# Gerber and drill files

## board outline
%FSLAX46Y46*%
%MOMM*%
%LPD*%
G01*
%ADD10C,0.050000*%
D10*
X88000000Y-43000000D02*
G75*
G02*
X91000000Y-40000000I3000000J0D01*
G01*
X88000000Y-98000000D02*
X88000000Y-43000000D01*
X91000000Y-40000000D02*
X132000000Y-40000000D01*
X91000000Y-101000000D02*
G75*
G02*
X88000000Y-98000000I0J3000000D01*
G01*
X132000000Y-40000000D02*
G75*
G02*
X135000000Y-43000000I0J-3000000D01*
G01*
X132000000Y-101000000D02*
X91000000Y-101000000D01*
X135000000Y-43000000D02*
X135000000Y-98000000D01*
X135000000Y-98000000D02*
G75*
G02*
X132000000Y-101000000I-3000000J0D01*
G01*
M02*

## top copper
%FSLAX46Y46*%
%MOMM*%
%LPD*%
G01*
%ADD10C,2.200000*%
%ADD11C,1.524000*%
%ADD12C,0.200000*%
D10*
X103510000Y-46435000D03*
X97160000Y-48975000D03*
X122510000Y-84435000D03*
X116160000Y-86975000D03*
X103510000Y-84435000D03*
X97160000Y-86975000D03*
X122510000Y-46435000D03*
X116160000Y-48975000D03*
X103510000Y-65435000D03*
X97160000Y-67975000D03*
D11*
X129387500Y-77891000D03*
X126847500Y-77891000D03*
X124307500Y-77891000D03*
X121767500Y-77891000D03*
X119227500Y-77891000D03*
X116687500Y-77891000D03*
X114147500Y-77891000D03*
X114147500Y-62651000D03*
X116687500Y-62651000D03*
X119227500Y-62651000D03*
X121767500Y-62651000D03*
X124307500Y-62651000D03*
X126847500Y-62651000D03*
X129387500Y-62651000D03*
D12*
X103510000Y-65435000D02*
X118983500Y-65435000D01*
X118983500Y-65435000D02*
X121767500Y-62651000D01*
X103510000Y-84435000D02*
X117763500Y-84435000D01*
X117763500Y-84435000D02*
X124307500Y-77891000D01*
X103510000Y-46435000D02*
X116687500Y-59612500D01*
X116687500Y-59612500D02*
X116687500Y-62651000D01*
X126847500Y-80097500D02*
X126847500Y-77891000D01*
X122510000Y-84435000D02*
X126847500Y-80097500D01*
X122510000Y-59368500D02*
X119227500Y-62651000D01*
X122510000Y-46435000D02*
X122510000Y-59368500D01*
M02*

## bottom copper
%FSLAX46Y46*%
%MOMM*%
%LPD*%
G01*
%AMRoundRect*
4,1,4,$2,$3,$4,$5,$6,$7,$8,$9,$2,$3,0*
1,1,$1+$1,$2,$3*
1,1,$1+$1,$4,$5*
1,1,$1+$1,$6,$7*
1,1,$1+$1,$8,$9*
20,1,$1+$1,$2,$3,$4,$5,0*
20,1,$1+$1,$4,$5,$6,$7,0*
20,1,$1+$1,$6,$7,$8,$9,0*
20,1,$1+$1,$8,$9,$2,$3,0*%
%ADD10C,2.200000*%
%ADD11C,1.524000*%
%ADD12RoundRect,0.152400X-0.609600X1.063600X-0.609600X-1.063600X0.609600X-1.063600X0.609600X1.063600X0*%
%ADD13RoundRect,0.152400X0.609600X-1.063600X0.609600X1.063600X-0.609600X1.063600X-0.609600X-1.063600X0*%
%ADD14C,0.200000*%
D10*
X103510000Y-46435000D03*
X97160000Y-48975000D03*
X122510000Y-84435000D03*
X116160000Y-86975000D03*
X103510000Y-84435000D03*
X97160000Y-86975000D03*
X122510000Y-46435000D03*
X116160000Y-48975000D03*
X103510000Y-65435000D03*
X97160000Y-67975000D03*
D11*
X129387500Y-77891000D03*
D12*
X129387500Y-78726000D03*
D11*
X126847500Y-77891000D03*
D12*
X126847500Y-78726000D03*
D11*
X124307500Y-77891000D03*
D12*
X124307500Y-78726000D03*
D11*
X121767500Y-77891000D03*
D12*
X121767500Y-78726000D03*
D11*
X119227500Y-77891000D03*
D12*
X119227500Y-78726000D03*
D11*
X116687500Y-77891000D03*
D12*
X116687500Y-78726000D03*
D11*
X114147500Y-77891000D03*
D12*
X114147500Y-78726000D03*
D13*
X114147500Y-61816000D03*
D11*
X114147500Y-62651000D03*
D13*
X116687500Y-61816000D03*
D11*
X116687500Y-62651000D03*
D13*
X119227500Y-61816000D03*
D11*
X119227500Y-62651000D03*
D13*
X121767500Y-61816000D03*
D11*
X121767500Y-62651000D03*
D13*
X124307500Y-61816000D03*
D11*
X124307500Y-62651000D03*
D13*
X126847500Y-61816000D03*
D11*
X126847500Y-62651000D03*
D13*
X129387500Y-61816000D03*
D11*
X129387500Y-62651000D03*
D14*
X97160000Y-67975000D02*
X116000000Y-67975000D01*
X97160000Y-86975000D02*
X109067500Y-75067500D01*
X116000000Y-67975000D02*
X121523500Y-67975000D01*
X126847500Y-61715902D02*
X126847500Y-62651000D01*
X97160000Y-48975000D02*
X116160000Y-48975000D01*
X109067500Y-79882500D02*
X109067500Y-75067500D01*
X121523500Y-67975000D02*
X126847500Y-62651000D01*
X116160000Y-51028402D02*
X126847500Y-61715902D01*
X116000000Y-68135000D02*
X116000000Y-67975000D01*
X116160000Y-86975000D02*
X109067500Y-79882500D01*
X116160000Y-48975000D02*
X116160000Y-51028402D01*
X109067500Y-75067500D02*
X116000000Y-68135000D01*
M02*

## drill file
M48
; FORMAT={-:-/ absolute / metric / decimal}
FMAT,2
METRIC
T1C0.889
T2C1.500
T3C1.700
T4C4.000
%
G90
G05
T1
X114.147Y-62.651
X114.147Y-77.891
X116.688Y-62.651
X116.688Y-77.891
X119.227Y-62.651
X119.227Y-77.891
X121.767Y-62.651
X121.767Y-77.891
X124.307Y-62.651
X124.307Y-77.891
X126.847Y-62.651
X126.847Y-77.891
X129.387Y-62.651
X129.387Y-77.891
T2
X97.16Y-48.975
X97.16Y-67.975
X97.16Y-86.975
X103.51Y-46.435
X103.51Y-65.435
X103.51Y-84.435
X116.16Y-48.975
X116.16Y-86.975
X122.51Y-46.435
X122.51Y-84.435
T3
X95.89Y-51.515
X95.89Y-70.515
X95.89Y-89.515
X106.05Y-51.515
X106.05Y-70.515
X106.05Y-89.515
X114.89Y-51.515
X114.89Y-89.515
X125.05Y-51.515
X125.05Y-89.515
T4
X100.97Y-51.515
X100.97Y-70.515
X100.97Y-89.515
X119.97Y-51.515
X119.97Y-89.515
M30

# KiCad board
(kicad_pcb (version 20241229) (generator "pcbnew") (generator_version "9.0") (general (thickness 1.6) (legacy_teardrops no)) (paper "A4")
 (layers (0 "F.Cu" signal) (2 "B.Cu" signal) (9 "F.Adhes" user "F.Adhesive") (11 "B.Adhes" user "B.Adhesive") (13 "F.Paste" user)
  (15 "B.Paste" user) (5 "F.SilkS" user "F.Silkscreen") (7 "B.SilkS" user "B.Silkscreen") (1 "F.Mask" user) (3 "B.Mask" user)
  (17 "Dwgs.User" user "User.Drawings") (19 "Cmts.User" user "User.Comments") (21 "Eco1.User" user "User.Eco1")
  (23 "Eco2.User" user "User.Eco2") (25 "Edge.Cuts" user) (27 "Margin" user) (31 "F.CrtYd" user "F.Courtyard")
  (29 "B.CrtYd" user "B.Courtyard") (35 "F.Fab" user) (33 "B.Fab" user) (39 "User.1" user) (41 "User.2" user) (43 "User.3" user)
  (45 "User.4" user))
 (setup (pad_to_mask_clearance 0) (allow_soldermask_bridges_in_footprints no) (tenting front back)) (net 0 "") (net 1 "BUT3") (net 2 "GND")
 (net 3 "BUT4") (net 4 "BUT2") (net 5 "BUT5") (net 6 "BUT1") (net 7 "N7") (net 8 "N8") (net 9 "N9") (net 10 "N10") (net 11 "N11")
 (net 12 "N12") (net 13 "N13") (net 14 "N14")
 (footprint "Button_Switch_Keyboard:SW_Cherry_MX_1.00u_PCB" (layer "F.Cu") (at 103.51 46.435)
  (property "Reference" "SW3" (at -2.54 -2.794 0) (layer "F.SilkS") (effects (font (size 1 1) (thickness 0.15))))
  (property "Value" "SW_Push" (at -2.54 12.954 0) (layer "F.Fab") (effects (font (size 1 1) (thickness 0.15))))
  (pad "" np_thru_hole circle (at -7.62 5.08) (size 1.7 1.7) (drill 1.7) (layers "*.Cu" "*.Mask"))
  (pad "" np_thru_hole circle (at -2.54 5.08) (size 4 4) (drill 4) (layers "*.Cu" "*.Mask"))
  (pad "" np_thru_hole circle (at 2.54 5.08) (size 1.7 1.7) (drill 1.7) (layers "*.Cu" "*.Mask"))
  (pad "1" thru_hole circle (at 0 0) (size 2.2 2.2) (drill 1.5) (layers "*.Cu" "*.Mask") (remove_unused_layers no) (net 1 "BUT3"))
  (pad "2" thru_hole circle (at -6.35 2.54) (size 2.2 2.2) (drill 1.5) (layers "*.Cu" "*.Mask") (remove_unused_layers no) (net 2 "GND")))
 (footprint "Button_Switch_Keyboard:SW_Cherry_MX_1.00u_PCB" (layer "F.Cu") (at 122.51 84.435)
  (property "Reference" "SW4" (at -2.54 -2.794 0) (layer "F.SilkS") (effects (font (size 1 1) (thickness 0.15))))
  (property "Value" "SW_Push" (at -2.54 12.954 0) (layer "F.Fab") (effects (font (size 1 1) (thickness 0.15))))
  (pad "" np_thru_hole circle (at -7.62 5.08) (size 1.7 1.7) (drill 1.7) (layers "*.Cu" "*.Mask"))
  (pad "" np_thru_hole circle (at -2.54 5.08) (size 4 4) (drill 4) (layers "*.Cu" "*.Mask"))
  (pad "" np_thru_hole circle (at 2.54 5.08) (size 1.7 1.7) (drill 1.7) (layers "*.Cu" "*.Mask"))
  (pad "1" thru_hole circle (at 0 0) (size 2.2 2.2) (drill 1.5) (layers "*.Cu" "*.Mask") (remove_unused_layers no) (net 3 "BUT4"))
  (pad "2" thru_hole circle (at -6.35 2.54) (size 2.2 2.2) (drill 1.5) (layers "*.Cu" "*.Mask") (remove_unused_layers no) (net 2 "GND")))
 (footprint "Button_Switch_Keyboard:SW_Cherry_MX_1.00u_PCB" (layer "F.Cu") (at 103.51 84.435)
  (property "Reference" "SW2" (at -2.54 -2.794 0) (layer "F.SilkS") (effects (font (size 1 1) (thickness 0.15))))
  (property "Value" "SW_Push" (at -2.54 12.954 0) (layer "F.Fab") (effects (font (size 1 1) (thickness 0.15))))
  (pad "" np_thru_hole circle (at -7.62 5.08) (size 1.7 1.7) (drill 1.7) (layers "*.Cu" "*.Mask"))
  (pad "" np_thru_hole circle (at -2.54 5.08) (size 4 4) (drill 4) (layers "*.Cu" "*.Mask"))
  (pad "" np_thru_hole circle (at 2.54 5.08) (size 1.7 1.7) (drill 1.7) (layers "*.Cu" "*.Mask"))
  (pad "1" thru_hole circle (at 0 0) (size 2.2 2.2) (drill 1.5) (layers "*.Cu" "*.Mask") (remove_unused_layers no) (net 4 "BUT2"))
  (pad "2" thru_hole circle (at -6.35 2.54) (size 2.2 2.2) (drill 1.5) (layers "*.Cu" "*.Mask") (remove_unused_layers no) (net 2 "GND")))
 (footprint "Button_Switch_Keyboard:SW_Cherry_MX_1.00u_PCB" (layer "F.Cu") (at 122.51 46.435)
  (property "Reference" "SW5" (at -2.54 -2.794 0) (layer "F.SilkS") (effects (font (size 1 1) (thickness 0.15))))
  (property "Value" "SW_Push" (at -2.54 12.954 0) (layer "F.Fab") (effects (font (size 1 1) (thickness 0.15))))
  (pad "" np_thru_hole circle (at -7.62 5.08) (size 1.7 1.7) (drill 1.7) (layers "*.Cu" "*.Mask"))
  (pad "" np_thru_hole circle (at -2.54 5.08) (size 4 4) (drill 4) (layers "*.Cu" "*.Mask"))
  (pad "" np_thru_hole circle (at 2.54 5.08) (size 1.7 1.7) (drill 1.7) (layers "*.Cu" "*.Mask"))
  (pad "1" thru_hole circle (at 0 0) (size 2.2 2.2) (drill 1.5) (layers "*.Cu" "*.Mask") (remove_unused_layers no) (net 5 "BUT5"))
  (pad "2" thru_hole circle (at -6.35 2.54) (size 2.2 2.2) (drill 1.5) (layers "*.Cu" "*.Mask") (remove_unused_layers no) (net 2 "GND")))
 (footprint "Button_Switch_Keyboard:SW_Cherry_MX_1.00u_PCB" (layer "F.Cu") (at 103.51 65.435)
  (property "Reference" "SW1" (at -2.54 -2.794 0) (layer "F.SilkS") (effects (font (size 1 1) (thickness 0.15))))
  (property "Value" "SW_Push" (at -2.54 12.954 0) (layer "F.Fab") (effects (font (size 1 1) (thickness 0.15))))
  (pad "" np_thru_hole circle (at -7.62 5.08) (size 1.7 1.7) (drill 1.7) (layers "*.Cu" "*.Mask"))
  (pad "" np_thru_hole circle (at -2.54 5.08) (size 4 4) (drill 4) (layers "*.Cu" "*.Mask"))
  (pad "" np_thru_hole circle (at 2.54 5.08) (size 1.7 1.7) (drill 1.7) (layers "*.Cu" "*.Mask"))
  (pad "1" thru_hole circle (at 0 0) (size 2.2 2.2) (drill 1.5) (layers "*.Cu" "*.Mask") (remove_unused_layers no) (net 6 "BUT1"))
  (pad "2" thru_hole circle (at -6.35 2.54) (size 2.2 2.2) (drill 1.5) (layers "*.Cu" "*.Mask") (remove_unused_layers no) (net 2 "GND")))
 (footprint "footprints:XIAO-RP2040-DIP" (layer "B.Cu") (at 121.7675 70.271)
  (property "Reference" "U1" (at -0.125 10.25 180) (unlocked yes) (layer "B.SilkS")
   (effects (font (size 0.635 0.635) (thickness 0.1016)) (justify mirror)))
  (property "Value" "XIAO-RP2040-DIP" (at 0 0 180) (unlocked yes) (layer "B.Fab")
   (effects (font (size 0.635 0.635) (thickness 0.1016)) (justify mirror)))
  (pad "1" thru_hole circle (at 7.62 7.62 270) (size 1.524 1.524) (drill 0.889) (layers "*.Cu" "*.Mask") (remove_unused_layers no)
   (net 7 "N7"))
  (pad "1" smd roundrect (at 7.62 8.455 270) (size 2.432 1.524) (layers "B.Cu" "B.Mask") (roundrect_rratio 0.1) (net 7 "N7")
   (thermal_bridge_angle 45))
  (pad "2" thru_hole circle (at 5.08 7.62 270) (size 1.524 1.524) (drill 0.889) (layers "*.Cu" "*.Mask") (remove_unused_layers no)
   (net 3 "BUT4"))
  (pad "2" smd roundrect (at 5.08 8.455 270) (size 2.432 1.524) (layers "B.Cu" "B.Mask") (roundrect_rratio 0.1) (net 3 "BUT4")
   (thermal_bridge_angle 45))
  (pad "3" thru_hole circle (at 2.54 7.62 270) (size 1.524 1.524) (drill 0.889) (layers "*.Cu" "*.Mask") (remove_unused_layers no)
   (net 4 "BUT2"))
  (pad "3" smd roundrect (at 2.54 8.455 270) (size 2.432 1.524) (layers "B.Cu" "B.Mask") (roundrect_rratio 0.1) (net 4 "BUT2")
   (thermal_bridge_angle 45))
  (pad "4" thru_hole circle (at 0 7.62 270) (size 1.524 1.524) (drill 0.889) (layers "*.Cu" "*.Mask") (remove_unused_layers no) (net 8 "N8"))
  (pad "4" smd roundrect (at 0 8.455 270) (size 2.432 1.524) (layers "B.Cu" "B.Mask") (roundrect_rratio 0.1) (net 8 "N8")
   (thermal_bridge_angle 45))
  (pad "5" thru_hole circle (at -2.54 7.62 270) (size 1.524 1.524) (drill 0.889) (layers "*.Cu" "*.Mask") (remove_unused_layers no)
   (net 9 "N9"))
  (pad "5" smd roundrect (at -2.54 8.455 270) (size 2.432 1.524) (layers "B.Cu" "B.Mask") (roundrect_rratio 0.1) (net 9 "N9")
   (thermal_bridge_angle 45))
  (pad "6" thru_hole circle (at -5.08 7.62 270) (size 1.524 1.524) (drill 0.889) (layers "*.Cu" "*.Mask") (remove_unused_layers no)
   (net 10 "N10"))
  (pad "6" smd roundrect (at -5.08 8.455 270) (size 2.432 1.524) (layers "B.Cu" "B.Mask") (roundrect_rratio 0.1) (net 10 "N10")
   (thermal_bridge_angle 45))
  (pad "7" thru_hole circle (at -7.62 7.62 270) (size 1.524 1.524) (drill 0.889) (layers "*.Cu" "*.Mask") (remove_unused_layers no)
   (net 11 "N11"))
  (pad "7" smd roundrect (at -7.62 8.455 270) (size 2.432 1.524) (layers "B.Cu" "B.Mask") (roundrect_rratio 0.1) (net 11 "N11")
   (thermal_bridge_angle 45))
  (pad "8" smd roundrect (at -7.62 -8.455 90) (size 2.432 1.524) (layers "B.Cu" "B.Mask") (roundrect_rratio 0.1) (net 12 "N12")
   (thermal_bridge_angle 45))
  (pad "8" thru_hole circle (at -7.62 -7.62 90) (size 1.524 1.524) (drill 0.889) (layers "*.Cu" "*.Mask") (remove_unused_layers no)
   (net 12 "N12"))
  (pad "9" smd roundrect (at -5.08 -8.455 90) (size 2.432 1.524) (layers "B.Cu" "B.Mask") (roundrect_rratio 0.1) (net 1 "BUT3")
   (thermal_bridge_angle 45))
  (pad "9" thru_hole circle (at -5.08 -7.62 90) (size 1.524 1.524) (drill 0.889) (layers "*.Cu" "*.Mask") (remove_unused_layers no)
   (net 1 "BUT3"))
  (pad "10" smd roundrect (at -2.54 -8.455 90) (size 2.432 1.524) (layers "B.Cu" "B.Mask") (roundrect_rratio 0.1) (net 5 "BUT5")
   (thermal_bridge_angle 45))
  (pad "10" thru_hole circle (at -2.54 -7.62 90) (size 1.524 1.524) (drill 0.889) (layers "*.Cu" "*.Mask") (remove_unused_layers no)
   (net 5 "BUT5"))
  (pad "11" smd roundrect (at 0 -8.455 90) (size 2.432 1.524) (layers "B.Cu" "B.Mask") (roundrect_rratio 0.1) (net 6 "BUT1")
   (thermal_bridge_angle 45))
  (pad "11" thru_hole circle (at 0 -7.62 90) (size 1.524 1.524) (drill 0.889) (layers "*.Cu" "*.Mask") (remove_unused_layers no)
   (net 6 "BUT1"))
  (pad "12" smd roundrect (at 2.54 -8.455 90) (size 2.432 1.524) (layers "B.Cu" "B.Mask") (roundrect_rratio 0.1) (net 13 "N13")
   (thermal_bridge_angle 45))
  (pad "12" thru_hole circle (at 2.54 -7.62 90) (size 1.524 1.524) (drill 0.889) (layers "*.Cu" "*.Mask") (remove_unused_layers no)
   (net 13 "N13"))
  (pad "13" smd roundrect (at 5.08 -8.455 90) (size 2.432 1.524) (layers "B.Cu" "B.Mask") (roundrect_rratio 0.1) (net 2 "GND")
   (thermal_bridge_angle 45))
  (pad "13" thru_hole circle (at 5.08 -7.62 90) (size 1.524 1.524) (drill 0.889) (layers "*.Cu" "*.Mask") (remove_unused_layers no)
   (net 2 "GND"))
  (pad "14" smd roundrect (at 7.62 -8.455 90) (size 2.432 1.524) (layers "B.Cu" "B.Mask") (roundrect_rratio 0.1) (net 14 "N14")
   (thermal_bridge_angle 45))
  (pad "14" thru_hole circle (at 7.62 -7.62 90) (size 1.524 1.524) (drill 0.889) (layers "*.Cu" "*.Mask") (remove_unused_layers no)
   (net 14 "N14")))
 (gr_arc (start 88 43) (mid 88.87868 40.87868) (end 91 40) (stroke (width 0.05) (type default)) (layer "Edge.Cuts"))
 (gr_line (start 88 98) (end 88 43) (stroke (width 0.05) (type default)) (layer "Edge.Cuts"))
 (gr_line (start 91 40) (end 132 40) (stroke (width 0.05) (type default)) (layer "Edge.Cuts"))
 (gr_arc (start 91 101) (mid 88.87868 100.12132) (end 88 98) (stroke (width 0.05) (type default)) (layer "Edge.Cuts"))
 (gr_arc (start 132 40) (mid 134.12132 40.87868) (end 135 43) (stroke (width 0.05) (type default)) (layer "Edge.Cuts"))
 (gr_line (start 132 101) (end 91 101) (stroke (width 0.05) (type default)) (layer "Edge.Cuts"))
 (gr_line (start 135 43) (end 135 98) (stroke (width 0.05) (type default)) (layer "Edge.Cuts"))
 (gr_arc (start 135 98) (mid 134.12132 100.12132) (end 132 101) (stroke (width 0.05) (type default)) (layer "Edge.Cuts"))
 (segment (start 103.51 65.435) (end 118.9835 65.435) (width 0.2) (layer "F.Cu") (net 6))
 (segment (start 118.9835 65.435) (end 121.7675 62.651) (width 0.2) (layer "F.Cu") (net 6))
 (segment (start 97.16 67.975) (end 116 67.975) (width 0.2) (layer "B.Cu") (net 2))
 (segment (start 97.16 86.975) (end 109.0675 75.0675) (width 0.2) (layer "B.Cu") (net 2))
 (segment (start 116 67.975) (end 121.5235 67.975) (width 0.2) (layer "B.Cu") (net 2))
 (segment (start 126.8475 61.715902) (end 126.8475 62.651) (width 0.2) (layer "B.Cu") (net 2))
 (segment (start 97.16 48.975) (end 116.16 48.975) (width 0.2) (layer "B.Cu") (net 2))
 (segment (start 109.0675 79.8825) (end 109.0675 75.0675) (width 0.2) (layer "B.Cu") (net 2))
 (segment (start 121.5235 67.975) (end 126.8475 62.651) (width 0.2) (layer "B.Cu") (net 2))
 (segment (start 116.16 51.028402) (end 126.8475 61.715902) (width 0.2) (layer "B.Cu") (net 2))
 (segment (start 116 68.135) (end 116 67.975) (width 0.2) (layer "B.Cu") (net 2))
 (segment (start 116.16 86.975) (end 109.0675 79.8825) (width 0.2) (layer "B.Cu") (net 2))
 (segment (start 116.16 48.975) (end 116.16 51.028402) (width 0.2) (layer "B.Cu") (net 2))
 (segment (start 109.0675 75.0675) (end 116 68.135) (width 0.2) (layer "B.Cu") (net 2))
 (segment (start 103.51 84.435) (end 117.7635 84.435) (width 0.2) (layer "F.Cu") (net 4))
 (segment (start 117.7635 84.435) (end 124.3075 77.891) (width 0.2) (layer "F.Cu") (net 4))
 (segment (start 103.51 46.435) (end 116.6875 59.6125) (width 0.2) (layer "F.Cu") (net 1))
 (segment (start 116.6875 59.6125) (end 116.6875 62.651) (width 0.2) (layer "F.Cu") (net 1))
 (segment (start 126.8475 80.0975) (end 126.8475 77.891) (width 0.2) (layer "F.Cu") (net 3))
 (segment (start 122.51 84.435) (end 126.8475 80.0975) (width 0.2) (layer "F.Cu") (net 3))
 (segment (start 122.51 59.3685) (end 119.2275 62.651) (width 0.2) (layer "F.Cu") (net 5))
 (segment (start 122.51 46.435) (end 122.51 59.3685) (width 0.2) (layer "F.Cu") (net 5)))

